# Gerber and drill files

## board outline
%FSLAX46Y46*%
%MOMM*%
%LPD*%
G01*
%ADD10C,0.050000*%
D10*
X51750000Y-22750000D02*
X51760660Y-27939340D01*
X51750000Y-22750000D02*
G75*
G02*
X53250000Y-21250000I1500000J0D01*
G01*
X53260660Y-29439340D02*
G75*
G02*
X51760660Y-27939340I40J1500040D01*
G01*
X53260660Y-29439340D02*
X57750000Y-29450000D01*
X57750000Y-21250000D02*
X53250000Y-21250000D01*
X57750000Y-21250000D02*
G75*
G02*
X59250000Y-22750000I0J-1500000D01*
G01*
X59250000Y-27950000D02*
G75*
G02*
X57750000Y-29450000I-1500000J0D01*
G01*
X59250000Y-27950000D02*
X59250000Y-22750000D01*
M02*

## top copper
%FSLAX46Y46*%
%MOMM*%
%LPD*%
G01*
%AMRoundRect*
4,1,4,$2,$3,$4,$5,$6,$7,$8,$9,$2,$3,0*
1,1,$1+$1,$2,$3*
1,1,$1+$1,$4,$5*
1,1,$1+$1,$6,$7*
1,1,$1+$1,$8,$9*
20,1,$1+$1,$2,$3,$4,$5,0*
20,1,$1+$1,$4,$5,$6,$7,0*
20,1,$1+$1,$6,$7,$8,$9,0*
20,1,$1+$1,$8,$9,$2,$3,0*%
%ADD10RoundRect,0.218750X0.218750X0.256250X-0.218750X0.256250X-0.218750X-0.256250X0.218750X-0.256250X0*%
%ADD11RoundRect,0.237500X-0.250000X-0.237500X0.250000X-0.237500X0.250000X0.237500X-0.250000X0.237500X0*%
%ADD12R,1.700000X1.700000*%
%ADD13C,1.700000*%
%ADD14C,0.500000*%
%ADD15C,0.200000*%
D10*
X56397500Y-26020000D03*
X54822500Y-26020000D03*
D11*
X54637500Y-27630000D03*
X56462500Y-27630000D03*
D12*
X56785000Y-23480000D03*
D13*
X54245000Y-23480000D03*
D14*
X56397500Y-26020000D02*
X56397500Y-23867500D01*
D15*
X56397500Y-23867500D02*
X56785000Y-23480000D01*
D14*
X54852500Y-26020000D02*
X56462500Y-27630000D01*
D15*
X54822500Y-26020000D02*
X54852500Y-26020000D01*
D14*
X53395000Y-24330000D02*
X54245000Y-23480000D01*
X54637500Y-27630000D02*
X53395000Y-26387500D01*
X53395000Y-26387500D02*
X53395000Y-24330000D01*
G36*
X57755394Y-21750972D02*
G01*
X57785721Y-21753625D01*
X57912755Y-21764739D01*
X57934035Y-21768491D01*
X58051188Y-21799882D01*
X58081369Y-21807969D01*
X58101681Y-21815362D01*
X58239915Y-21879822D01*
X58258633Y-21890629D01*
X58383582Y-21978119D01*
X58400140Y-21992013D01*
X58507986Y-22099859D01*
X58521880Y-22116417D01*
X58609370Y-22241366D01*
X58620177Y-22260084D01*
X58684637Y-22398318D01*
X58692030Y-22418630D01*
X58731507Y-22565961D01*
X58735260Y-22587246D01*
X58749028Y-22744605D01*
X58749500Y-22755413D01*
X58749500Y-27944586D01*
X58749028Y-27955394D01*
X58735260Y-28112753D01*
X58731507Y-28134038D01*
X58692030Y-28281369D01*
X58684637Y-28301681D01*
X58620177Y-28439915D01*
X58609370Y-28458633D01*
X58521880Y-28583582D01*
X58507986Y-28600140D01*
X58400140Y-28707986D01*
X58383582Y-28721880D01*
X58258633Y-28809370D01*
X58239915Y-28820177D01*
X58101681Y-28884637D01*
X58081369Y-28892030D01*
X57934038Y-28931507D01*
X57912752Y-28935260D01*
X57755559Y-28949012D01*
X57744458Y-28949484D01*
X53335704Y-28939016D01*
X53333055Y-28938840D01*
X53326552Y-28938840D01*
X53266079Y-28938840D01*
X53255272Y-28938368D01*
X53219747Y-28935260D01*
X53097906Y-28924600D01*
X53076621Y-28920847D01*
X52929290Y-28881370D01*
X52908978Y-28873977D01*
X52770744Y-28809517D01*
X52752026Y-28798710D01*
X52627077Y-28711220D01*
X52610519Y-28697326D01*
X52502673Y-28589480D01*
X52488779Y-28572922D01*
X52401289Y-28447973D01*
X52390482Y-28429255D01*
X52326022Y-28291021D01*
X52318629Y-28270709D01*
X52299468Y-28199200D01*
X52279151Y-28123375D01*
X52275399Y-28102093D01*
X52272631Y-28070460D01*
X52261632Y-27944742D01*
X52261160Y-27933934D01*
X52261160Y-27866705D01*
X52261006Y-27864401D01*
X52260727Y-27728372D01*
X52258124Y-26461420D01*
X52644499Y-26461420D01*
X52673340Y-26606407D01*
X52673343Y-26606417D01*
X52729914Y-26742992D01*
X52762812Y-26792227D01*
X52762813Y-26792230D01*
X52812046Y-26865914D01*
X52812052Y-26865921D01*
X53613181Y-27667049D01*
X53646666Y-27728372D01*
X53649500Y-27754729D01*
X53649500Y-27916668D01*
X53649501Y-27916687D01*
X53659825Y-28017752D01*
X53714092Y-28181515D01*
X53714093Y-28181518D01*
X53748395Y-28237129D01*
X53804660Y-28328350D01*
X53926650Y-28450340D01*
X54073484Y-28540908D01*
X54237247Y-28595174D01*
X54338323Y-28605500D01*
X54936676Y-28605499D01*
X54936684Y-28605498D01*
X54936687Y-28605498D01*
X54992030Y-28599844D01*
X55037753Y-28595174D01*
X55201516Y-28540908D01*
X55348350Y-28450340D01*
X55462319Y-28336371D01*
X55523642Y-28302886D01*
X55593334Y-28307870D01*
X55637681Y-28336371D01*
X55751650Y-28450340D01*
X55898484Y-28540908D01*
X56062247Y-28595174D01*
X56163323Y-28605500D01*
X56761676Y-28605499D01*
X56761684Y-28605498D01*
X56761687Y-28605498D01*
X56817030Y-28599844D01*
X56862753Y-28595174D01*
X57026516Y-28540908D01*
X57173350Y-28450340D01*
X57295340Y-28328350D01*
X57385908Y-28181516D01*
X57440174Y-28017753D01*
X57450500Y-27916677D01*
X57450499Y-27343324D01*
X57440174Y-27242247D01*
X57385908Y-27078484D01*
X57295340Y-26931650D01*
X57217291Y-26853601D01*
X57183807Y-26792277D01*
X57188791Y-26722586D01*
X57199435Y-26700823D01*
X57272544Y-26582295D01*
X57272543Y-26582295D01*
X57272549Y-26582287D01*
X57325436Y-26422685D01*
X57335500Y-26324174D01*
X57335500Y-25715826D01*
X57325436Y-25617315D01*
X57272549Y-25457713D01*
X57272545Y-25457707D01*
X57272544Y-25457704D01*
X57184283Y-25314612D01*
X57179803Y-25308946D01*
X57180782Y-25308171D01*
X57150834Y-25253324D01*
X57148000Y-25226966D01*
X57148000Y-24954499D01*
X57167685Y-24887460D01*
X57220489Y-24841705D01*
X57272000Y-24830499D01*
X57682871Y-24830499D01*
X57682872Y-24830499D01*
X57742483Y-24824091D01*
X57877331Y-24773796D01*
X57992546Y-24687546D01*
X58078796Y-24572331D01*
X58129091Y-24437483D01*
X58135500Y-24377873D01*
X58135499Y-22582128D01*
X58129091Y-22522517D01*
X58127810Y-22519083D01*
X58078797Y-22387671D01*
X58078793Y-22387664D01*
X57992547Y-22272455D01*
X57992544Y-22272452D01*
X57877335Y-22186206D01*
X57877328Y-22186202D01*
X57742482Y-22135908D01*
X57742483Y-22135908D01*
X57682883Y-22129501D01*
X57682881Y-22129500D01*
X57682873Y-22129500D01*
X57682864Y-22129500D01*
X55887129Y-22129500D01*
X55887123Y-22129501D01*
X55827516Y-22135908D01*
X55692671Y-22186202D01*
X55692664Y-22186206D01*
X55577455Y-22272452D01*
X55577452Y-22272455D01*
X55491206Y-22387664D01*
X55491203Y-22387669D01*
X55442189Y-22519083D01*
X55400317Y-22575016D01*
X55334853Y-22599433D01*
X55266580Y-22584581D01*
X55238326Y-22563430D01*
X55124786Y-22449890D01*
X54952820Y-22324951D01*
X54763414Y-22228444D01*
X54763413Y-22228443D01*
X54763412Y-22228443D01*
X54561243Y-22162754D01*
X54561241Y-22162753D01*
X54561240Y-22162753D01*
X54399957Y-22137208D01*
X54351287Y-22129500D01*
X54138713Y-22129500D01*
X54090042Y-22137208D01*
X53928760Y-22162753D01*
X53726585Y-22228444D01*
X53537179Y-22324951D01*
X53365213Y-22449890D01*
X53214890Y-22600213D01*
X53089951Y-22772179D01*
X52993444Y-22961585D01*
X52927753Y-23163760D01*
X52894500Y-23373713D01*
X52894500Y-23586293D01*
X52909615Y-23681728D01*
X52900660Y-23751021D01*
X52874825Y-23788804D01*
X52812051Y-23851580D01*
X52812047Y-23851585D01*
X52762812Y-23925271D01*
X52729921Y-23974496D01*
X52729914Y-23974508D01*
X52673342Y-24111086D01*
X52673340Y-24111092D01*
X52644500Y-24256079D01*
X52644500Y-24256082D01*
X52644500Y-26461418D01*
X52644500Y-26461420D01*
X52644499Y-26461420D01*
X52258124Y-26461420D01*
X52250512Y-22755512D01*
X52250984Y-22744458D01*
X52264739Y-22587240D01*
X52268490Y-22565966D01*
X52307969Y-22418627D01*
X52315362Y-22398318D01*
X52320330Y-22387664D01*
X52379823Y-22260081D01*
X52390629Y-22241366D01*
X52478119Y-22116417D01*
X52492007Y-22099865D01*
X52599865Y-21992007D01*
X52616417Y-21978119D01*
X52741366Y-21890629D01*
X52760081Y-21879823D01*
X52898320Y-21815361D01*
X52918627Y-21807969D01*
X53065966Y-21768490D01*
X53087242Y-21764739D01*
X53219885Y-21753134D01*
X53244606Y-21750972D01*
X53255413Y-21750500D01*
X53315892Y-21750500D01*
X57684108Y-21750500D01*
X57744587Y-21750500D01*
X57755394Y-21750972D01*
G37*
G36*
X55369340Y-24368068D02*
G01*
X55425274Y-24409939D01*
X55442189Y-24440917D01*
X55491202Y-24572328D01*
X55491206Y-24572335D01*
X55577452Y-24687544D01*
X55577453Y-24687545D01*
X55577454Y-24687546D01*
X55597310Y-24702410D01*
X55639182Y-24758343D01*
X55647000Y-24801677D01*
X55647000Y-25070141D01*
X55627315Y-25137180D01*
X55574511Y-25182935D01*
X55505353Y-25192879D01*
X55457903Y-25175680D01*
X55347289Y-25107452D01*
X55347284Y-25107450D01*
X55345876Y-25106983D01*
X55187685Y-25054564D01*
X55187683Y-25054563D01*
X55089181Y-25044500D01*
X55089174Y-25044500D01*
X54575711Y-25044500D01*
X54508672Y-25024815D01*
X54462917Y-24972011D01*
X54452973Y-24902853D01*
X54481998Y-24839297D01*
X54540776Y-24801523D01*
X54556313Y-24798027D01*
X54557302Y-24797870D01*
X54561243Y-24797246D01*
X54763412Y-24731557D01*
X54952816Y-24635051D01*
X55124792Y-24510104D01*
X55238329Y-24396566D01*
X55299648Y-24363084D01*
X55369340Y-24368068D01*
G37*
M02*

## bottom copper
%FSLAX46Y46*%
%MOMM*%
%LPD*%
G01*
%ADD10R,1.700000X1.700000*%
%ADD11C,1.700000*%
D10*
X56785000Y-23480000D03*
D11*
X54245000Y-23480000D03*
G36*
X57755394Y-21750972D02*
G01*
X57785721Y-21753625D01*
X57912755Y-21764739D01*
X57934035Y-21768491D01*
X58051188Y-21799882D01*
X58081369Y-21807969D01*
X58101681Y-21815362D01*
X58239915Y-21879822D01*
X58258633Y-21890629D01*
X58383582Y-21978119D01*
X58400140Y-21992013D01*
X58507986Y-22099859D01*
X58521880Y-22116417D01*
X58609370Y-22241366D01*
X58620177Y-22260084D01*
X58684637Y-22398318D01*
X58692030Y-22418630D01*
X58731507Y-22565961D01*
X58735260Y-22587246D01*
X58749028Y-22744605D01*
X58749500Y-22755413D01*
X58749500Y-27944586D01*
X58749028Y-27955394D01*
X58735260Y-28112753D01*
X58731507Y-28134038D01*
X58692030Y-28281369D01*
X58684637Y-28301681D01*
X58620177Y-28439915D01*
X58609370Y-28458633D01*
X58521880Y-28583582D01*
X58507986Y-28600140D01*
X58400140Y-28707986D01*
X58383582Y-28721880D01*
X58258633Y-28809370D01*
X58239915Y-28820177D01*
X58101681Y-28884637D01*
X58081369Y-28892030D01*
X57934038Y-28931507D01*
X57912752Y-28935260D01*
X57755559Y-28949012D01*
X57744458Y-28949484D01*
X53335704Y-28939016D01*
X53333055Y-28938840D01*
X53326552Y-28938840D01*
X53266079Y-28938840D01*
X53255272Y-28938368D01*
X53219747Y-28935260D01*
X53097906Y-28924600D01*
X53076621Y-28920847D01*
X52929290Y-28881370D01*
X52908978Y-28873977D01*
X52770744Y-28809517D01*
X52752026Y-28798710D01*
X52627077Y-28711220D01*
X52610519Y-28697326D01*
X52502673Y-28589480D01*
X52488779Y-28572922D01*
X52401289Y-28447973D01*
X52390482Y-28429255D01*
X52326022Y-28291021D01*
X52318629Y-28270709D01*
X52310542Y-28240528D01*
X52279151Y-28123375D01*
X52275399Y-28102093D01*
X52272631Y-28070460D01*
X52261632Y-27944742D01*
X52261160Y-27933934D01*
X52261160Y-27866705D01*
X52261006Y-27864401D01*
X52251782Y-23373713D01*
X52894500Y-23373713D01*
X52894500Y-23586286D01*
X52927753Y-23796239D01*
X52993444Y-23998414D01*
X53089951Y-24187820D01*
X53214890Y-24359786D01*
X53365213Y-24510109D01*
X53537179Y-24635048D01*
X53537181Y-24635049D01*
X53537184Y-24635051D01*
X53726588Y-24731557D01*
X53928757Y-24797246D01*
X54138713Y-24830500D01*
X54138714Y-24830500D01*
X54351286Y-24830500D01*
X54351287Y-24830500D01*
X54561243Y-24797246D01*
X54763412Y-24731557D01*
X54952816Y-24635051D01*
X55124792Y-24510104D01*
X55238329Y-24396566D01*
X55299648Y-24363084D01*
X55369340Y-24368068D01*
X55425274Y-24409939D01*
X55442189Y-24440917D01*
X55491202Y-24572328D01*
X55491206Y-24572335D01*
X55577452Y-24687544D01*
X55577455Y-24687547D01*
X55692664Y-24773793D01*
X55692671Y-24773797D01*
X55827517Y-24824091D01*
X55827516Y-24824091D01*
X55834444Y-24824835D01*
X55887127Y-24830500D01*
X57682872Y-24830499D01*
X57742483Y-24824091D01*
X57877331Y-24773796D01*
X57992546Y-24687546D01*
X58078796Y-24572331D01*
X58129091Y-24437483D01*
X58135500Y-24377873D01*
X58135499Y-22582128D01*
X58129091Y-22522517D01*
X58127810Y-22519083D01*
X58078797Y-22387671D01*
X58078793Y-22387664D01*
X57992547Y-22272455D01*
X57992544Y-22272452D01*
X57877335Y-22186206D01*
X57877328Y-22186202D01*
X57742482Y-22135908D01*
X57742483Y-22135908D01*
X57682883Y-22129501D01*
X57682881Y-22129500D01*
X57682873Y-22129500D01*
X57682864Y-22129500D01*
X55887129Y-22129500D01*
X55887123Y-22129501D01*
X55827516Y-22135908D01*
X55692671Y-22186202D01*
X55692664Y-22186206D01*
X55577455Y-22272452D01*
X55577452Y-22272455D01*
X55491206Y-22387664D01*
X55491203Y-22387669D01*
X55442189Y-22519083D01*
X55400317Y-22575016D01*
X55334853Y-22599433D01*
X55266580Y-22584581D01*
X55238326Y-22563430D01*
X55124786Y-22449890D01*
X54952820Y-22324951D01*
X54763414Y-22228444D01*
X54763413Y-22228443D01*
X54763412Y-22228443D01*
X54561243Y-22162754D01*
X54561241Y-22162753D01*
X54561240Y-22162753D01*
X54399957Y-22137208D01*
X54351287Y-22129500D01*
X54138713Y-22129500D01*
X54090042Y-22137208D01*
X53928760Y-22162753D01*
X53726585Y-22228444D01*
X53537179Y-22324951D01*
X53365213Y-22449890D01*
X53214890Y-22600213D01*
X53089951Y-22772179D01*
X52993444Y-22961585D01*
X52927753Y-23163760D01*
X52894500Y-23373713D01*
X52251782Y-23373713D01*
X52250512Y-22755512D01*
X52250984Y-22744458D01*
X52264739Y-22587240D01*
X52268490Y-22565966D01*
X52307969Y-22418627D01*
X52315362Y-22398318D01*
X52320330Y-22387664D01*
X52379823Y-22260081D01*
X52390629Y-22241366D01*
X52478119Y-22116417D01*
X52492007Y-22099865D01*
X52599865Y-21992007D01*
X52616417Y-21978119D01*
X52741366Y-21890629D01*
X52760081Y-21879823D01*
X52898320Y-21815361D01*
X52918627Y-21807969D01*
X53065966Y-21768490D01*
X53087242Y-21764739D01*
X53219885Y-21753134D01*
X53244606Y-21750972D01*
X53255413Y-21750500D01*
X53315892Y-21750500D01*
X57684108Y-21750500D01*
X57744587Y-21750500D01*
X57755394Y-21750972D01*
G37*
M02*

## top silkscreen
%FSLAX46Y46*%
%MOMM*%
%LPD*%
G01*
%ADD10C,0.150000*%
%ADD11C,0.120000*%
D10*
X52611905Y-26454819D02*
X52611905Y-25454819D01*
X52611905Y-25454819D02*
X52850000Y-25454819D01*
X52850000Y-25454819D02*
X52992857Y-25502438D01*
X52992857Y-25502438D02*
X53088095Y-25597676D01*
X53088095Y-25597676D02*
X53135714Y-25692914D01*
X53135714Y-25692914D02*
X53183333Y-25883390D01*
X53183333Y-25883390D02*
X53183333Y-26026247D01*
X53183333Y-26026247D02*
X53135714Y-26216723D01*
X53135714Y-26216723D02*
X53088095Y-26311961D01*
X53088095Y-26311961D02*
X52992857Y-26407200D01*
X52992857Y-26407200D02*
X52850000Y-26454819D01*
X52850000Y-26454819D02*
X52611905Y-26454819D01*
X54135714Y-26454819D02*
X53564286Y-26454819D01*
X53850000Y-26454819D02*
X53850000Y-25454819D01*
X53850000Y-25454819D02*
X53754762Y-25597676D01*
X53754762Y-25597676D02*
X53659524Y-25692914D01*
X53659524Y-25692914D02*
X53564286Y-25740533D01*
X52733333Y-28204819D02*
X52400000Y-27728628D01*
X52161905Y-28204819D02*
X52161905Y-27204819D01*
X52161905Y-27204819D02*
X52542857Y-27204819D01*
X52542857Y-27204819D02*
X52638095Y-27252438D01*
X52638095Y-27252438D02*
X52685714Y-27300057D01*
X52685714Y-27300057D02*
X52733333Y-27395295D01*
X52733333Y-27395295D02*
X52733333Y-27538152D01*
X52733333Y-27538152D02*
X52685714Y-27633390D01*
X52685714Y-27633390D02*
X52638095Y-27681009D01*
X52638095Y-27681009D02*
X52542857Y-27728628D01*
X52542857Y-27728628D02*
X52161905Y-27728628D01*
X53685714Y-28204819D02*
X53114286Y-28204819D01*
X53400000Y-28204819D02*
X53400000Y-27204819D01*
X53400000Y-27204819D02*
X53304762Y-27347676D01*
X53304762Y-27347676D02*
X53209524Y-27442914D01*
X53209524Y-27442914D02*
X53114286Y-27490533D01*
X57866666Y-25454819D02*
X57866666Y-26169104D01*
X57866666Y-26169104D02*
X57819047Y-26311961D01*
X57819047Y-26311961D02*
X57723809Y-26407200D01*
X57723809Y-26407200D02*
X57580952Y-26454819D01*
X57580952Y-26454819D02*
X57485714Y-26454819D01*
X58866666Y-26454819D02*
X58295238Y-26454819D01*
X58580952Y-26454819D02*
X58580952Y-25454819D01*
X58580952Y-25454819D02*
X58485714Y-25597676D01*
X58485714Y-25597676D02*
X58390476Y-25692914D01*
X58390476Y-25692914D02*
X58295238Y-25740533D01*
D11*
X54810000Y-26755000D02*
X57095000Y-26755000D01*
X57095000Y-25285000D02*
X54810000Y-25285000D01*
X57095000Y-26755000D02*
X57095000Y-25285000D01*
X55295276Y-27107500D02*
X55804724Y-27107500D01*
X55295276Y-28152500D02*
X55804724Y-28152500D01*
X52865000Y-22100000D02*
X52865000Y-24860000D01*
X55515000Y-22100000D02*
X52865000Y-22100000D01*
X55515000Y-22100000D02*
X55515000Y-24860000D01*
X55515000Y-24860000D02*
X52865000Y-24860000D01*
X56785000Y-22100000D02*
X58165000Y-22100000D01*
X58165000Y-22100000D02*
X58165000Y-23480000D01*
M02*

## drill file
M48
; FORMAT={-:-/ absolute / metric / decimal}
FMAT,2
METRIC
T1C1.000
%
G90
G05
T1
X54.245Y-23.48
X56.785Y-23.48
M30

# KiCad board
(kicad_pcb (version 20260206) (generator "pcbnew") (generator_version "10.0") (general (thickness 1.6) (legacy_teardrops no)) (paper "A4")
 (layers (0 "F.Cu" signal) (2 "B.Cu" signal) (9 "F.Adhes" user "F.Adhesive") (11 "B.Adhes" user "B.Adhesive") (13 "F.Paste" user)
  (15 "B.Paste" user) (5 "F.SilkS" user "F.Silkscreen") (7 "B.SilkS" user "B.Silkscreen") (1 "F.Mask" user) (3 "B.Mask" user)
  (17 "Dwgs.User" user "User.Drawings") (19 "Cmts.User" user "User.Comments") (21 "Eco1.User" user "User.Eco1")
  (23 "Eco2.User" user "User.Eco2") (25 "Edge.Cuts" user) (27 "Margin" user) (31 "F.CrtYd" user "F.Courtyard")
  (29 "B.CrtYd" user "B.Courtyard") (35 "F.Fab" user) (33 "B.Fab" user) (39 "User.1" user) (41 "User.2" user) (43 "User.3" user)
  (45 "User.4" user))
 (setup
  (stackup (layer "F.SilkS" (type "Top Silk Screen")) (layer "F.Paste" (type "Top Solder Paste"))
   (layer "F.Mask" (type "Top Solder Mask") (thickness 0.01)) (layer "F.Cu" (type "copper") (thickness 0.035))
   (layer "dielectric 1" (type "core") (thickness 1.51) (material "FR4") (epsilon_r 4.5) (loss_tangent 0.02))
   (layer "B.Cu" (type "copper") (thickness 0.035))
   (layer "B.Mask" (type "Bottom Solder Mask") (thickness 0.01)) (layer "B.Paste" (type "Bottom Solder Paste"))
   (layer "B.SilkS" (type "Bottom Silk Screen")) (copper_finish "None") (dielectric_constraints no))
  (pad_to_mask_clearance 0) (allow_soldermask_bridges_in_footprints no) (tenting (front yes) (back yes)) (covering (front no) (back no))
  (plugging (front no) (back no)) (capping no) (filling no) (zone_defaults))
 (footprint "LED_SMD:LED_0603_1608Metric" (layer "F.Cu") (at 55.61 26.02 180)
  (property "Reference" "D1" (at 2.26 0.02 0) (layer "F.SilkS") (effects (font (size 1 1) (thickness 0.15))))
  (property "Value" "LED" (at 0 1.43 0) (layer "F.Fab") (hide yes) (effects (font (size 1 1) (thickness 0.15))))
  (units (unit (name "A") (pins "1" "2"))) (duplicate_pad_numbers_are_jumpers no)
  (fp_line (start 0.8 -0.735) (end -1.485 -0.735) (stroke (width 0.12) (type solid)) (layer "F.SilkS"))
  (fp_line (start -1.485 0.735) (end 0.8 0.735) (stroke (width 0.12) (type solid)) (layer "F.SilkS"))
  (fp_line (start -1.485 -0.735) (end -1.485 0.735) (stroke (width 0.12) (type solid)) (layer "F.SilkS"))
  (pad "1" smd roundrect (at -0.7875 0 180) (size 0.875 0.95) (layers "F.Cu" "F.Mask" "F.Paste") (roundrect_rratio 0.25) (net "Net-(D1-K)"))
  (pad "2" smd roundrect (at 0.7875 0 180) (size 0.875 0.95) (layers "F.Cu" "F.Mask" "F.Paste") (roundrect_rratio 0.25) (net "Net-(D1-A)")))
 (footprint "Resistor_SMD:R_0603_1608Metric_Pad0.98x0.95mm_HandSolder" (layer "F.Cu") (at 55.55 27.63)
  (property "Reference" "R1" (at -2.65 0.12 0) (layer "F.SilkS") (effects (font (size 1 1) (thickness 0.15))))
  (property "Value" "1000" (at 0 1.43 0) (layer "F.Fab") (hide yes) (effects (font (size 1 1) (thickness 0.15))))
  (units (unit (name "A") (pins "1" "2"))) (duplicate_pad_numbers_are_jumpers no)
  (fp_line (start -0.254724 -0.5225) (end 0.254724 -0.5225) (stroke (width 0.12) (type solid)) (layer "F.SilkS"))
  (fp_line (start -0.254724 0.5225) (end 0.254724 0.5225) (stroke (width 0.12) (type solid)) (layer "F.SilkS"))
  (pad "1" smd roundrect (at -0.9125 0) (size 0.975 0.95) (layers "F.Cu" "F.Mask" "F.Paste") (roundrect_rratio 0.25) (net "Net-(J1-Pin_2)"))
  (pad "2" smd roundrect (at 0.9125 0) (size 0.975 0.95) (layers "F.Cu" "F.Mask" "F.Paste") (roundrect_rratio 0.25) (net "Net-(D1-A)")))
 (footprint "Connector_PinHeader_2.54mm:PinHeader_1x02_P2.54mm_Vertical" (layer "F.Cu") (at 56.785 23.48 -90)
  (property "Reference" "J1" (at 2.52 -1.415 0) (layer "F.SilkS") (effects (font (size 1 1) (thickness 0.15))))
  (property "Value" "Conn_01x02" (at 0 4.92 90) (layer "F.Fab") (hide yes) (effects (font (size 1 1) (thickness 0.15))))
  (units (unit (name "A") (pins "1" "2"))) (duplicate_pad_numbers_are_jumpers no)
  (fp_line (start -1.38 3.92) (end 1.38 3.92) (stroke (width 0.12) (type solid)) (layer "F.SilkS"))
  (fp_line (start -1.38 1.27) (end -1.38 3.92) (stroke (width 0.12) (type solid)) (layer "F.SilkS"))
  (fp_line (start -1.38 1.27) (end 1.38 1.27) (stroke (width 0.12) (type solid)) (layer "F.SilkS"))
  (fp_line (start 1.38 1.27) (end 1.38 3.92) (stroke (width 0.12) (type solid)) (layer "F.SilkS"))
  (fp_line (start -1.38 0) (end -1.38 -1.38) (stroke (width 0.12) (type solid)) (layer "F.SilkS"))
  (fp_line (start -1.38 -1.38) (end 0 -1.38) (stroke (width 0.12) (type solid)) (layer "F.SilkS"))
  (pad "1" thru_hole rect (at 0 0 270) (size 1.7 1.7) (drill 1) (layers "*.Cu" "*.Mask") (remove_unused_layers no) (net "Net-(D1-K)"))
  (pad "2" thru_hole circle (at 0 2.54 270) (size 1.7 1.7) (drill 1) (layers "*.Cu" "*.Mask") (remove_unused_layers no)
   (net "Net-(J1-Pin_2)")))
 (gr_line (start 51.75 22.75) (end 51.76066 27.93934) (stroke (width 0.05) (type default)) (layer "Edge.Cuts"))
 (gr_arc (start 51.75 22.75) (mid 52.18934 21.68934) (end 53.25 21.25) (stroke (width 0.05) (type default)) (layer "Edge.Cuts"))
 (gr_arc (start 53.26066 29.43934) (mid 52.2 29) (end 51.76066 27.93934) (stroke (width 0.05) (type default)) (layer "Edge.Cuts"))
 (gr_line (start 53.26066 29.43934) (end 57.75 29.45) (stroke (width 0.05) (type default)) (layer "Edge.Cuts"))
 (gr_line (start 57.75 21.25) (end 53.25 21.25) (stroke (width 0.05) (type default)) (layer "Edge.Cuts"))
 (gr_arc (start 57.75 21.25) (mid 58.81066 21.68934) (end 59.25 22.75) (stroke (width 0.05) (type default)) (layer "Edge.Cuts"))
 (gr_arc (start 59.25 27.95) (mid 58.81066 29.01066) (end 57.75 29.45) (stroke (width 0.05) (type default)) (layer "Edge.Cuts"))
 (gr_line (start 59.25 27.95) (end 59.25 22.75) (stroke (width 0.05) (type default)) (layer "Edge.Cuts"))
 (segment (start 56.3975 26.02) (end 56.3975 23.8675) (width 0.5) (layer "F.Cu") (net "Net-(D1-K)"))
 (segment (start 56.3975 23.8675) (end 56.785 23.48) (width 0.2) (layer "F.Cu") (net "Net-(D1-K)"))
 (segment (start 54.8525 26.02) (end 56.4625 27.63) (width 0.5) (layer "F.Cu") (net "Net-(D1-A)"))
 (segment (start 54.8225 26.02) (end 54.8525 26.02) (width 0.2) (layer "F.Cu") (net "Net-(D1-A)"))
 (segment (start 53.395 24.33) (end 54.245 23.48) (width 0.5) (layer "F.Cu") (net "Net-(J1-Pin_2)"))
 (segment (start 54.6375 27.63) (end 53.395 26.3875) (width 0.5) (layer "F.Cu") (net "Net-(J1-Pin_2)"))
 (segment (start 53.395 26.3875) (end 53.395 24.33) (width 0.5) (layer "F.Cu") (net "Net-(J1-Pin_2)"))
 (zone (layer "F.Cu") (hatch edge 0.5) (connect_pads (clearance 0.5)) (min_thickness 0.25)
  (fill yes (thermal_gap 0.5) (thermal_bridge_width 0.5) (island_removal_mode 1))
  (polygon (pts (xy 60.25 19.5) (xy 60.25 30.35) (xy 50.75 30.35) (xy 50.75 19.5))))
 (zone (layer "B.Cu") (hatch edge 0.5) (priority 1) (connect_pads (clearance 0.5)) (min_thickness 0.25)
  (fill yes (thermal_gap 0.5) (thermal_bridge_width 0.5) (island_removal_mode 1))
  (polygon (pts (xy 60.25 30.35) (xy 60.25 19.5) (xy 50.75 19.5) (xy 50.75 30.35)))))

